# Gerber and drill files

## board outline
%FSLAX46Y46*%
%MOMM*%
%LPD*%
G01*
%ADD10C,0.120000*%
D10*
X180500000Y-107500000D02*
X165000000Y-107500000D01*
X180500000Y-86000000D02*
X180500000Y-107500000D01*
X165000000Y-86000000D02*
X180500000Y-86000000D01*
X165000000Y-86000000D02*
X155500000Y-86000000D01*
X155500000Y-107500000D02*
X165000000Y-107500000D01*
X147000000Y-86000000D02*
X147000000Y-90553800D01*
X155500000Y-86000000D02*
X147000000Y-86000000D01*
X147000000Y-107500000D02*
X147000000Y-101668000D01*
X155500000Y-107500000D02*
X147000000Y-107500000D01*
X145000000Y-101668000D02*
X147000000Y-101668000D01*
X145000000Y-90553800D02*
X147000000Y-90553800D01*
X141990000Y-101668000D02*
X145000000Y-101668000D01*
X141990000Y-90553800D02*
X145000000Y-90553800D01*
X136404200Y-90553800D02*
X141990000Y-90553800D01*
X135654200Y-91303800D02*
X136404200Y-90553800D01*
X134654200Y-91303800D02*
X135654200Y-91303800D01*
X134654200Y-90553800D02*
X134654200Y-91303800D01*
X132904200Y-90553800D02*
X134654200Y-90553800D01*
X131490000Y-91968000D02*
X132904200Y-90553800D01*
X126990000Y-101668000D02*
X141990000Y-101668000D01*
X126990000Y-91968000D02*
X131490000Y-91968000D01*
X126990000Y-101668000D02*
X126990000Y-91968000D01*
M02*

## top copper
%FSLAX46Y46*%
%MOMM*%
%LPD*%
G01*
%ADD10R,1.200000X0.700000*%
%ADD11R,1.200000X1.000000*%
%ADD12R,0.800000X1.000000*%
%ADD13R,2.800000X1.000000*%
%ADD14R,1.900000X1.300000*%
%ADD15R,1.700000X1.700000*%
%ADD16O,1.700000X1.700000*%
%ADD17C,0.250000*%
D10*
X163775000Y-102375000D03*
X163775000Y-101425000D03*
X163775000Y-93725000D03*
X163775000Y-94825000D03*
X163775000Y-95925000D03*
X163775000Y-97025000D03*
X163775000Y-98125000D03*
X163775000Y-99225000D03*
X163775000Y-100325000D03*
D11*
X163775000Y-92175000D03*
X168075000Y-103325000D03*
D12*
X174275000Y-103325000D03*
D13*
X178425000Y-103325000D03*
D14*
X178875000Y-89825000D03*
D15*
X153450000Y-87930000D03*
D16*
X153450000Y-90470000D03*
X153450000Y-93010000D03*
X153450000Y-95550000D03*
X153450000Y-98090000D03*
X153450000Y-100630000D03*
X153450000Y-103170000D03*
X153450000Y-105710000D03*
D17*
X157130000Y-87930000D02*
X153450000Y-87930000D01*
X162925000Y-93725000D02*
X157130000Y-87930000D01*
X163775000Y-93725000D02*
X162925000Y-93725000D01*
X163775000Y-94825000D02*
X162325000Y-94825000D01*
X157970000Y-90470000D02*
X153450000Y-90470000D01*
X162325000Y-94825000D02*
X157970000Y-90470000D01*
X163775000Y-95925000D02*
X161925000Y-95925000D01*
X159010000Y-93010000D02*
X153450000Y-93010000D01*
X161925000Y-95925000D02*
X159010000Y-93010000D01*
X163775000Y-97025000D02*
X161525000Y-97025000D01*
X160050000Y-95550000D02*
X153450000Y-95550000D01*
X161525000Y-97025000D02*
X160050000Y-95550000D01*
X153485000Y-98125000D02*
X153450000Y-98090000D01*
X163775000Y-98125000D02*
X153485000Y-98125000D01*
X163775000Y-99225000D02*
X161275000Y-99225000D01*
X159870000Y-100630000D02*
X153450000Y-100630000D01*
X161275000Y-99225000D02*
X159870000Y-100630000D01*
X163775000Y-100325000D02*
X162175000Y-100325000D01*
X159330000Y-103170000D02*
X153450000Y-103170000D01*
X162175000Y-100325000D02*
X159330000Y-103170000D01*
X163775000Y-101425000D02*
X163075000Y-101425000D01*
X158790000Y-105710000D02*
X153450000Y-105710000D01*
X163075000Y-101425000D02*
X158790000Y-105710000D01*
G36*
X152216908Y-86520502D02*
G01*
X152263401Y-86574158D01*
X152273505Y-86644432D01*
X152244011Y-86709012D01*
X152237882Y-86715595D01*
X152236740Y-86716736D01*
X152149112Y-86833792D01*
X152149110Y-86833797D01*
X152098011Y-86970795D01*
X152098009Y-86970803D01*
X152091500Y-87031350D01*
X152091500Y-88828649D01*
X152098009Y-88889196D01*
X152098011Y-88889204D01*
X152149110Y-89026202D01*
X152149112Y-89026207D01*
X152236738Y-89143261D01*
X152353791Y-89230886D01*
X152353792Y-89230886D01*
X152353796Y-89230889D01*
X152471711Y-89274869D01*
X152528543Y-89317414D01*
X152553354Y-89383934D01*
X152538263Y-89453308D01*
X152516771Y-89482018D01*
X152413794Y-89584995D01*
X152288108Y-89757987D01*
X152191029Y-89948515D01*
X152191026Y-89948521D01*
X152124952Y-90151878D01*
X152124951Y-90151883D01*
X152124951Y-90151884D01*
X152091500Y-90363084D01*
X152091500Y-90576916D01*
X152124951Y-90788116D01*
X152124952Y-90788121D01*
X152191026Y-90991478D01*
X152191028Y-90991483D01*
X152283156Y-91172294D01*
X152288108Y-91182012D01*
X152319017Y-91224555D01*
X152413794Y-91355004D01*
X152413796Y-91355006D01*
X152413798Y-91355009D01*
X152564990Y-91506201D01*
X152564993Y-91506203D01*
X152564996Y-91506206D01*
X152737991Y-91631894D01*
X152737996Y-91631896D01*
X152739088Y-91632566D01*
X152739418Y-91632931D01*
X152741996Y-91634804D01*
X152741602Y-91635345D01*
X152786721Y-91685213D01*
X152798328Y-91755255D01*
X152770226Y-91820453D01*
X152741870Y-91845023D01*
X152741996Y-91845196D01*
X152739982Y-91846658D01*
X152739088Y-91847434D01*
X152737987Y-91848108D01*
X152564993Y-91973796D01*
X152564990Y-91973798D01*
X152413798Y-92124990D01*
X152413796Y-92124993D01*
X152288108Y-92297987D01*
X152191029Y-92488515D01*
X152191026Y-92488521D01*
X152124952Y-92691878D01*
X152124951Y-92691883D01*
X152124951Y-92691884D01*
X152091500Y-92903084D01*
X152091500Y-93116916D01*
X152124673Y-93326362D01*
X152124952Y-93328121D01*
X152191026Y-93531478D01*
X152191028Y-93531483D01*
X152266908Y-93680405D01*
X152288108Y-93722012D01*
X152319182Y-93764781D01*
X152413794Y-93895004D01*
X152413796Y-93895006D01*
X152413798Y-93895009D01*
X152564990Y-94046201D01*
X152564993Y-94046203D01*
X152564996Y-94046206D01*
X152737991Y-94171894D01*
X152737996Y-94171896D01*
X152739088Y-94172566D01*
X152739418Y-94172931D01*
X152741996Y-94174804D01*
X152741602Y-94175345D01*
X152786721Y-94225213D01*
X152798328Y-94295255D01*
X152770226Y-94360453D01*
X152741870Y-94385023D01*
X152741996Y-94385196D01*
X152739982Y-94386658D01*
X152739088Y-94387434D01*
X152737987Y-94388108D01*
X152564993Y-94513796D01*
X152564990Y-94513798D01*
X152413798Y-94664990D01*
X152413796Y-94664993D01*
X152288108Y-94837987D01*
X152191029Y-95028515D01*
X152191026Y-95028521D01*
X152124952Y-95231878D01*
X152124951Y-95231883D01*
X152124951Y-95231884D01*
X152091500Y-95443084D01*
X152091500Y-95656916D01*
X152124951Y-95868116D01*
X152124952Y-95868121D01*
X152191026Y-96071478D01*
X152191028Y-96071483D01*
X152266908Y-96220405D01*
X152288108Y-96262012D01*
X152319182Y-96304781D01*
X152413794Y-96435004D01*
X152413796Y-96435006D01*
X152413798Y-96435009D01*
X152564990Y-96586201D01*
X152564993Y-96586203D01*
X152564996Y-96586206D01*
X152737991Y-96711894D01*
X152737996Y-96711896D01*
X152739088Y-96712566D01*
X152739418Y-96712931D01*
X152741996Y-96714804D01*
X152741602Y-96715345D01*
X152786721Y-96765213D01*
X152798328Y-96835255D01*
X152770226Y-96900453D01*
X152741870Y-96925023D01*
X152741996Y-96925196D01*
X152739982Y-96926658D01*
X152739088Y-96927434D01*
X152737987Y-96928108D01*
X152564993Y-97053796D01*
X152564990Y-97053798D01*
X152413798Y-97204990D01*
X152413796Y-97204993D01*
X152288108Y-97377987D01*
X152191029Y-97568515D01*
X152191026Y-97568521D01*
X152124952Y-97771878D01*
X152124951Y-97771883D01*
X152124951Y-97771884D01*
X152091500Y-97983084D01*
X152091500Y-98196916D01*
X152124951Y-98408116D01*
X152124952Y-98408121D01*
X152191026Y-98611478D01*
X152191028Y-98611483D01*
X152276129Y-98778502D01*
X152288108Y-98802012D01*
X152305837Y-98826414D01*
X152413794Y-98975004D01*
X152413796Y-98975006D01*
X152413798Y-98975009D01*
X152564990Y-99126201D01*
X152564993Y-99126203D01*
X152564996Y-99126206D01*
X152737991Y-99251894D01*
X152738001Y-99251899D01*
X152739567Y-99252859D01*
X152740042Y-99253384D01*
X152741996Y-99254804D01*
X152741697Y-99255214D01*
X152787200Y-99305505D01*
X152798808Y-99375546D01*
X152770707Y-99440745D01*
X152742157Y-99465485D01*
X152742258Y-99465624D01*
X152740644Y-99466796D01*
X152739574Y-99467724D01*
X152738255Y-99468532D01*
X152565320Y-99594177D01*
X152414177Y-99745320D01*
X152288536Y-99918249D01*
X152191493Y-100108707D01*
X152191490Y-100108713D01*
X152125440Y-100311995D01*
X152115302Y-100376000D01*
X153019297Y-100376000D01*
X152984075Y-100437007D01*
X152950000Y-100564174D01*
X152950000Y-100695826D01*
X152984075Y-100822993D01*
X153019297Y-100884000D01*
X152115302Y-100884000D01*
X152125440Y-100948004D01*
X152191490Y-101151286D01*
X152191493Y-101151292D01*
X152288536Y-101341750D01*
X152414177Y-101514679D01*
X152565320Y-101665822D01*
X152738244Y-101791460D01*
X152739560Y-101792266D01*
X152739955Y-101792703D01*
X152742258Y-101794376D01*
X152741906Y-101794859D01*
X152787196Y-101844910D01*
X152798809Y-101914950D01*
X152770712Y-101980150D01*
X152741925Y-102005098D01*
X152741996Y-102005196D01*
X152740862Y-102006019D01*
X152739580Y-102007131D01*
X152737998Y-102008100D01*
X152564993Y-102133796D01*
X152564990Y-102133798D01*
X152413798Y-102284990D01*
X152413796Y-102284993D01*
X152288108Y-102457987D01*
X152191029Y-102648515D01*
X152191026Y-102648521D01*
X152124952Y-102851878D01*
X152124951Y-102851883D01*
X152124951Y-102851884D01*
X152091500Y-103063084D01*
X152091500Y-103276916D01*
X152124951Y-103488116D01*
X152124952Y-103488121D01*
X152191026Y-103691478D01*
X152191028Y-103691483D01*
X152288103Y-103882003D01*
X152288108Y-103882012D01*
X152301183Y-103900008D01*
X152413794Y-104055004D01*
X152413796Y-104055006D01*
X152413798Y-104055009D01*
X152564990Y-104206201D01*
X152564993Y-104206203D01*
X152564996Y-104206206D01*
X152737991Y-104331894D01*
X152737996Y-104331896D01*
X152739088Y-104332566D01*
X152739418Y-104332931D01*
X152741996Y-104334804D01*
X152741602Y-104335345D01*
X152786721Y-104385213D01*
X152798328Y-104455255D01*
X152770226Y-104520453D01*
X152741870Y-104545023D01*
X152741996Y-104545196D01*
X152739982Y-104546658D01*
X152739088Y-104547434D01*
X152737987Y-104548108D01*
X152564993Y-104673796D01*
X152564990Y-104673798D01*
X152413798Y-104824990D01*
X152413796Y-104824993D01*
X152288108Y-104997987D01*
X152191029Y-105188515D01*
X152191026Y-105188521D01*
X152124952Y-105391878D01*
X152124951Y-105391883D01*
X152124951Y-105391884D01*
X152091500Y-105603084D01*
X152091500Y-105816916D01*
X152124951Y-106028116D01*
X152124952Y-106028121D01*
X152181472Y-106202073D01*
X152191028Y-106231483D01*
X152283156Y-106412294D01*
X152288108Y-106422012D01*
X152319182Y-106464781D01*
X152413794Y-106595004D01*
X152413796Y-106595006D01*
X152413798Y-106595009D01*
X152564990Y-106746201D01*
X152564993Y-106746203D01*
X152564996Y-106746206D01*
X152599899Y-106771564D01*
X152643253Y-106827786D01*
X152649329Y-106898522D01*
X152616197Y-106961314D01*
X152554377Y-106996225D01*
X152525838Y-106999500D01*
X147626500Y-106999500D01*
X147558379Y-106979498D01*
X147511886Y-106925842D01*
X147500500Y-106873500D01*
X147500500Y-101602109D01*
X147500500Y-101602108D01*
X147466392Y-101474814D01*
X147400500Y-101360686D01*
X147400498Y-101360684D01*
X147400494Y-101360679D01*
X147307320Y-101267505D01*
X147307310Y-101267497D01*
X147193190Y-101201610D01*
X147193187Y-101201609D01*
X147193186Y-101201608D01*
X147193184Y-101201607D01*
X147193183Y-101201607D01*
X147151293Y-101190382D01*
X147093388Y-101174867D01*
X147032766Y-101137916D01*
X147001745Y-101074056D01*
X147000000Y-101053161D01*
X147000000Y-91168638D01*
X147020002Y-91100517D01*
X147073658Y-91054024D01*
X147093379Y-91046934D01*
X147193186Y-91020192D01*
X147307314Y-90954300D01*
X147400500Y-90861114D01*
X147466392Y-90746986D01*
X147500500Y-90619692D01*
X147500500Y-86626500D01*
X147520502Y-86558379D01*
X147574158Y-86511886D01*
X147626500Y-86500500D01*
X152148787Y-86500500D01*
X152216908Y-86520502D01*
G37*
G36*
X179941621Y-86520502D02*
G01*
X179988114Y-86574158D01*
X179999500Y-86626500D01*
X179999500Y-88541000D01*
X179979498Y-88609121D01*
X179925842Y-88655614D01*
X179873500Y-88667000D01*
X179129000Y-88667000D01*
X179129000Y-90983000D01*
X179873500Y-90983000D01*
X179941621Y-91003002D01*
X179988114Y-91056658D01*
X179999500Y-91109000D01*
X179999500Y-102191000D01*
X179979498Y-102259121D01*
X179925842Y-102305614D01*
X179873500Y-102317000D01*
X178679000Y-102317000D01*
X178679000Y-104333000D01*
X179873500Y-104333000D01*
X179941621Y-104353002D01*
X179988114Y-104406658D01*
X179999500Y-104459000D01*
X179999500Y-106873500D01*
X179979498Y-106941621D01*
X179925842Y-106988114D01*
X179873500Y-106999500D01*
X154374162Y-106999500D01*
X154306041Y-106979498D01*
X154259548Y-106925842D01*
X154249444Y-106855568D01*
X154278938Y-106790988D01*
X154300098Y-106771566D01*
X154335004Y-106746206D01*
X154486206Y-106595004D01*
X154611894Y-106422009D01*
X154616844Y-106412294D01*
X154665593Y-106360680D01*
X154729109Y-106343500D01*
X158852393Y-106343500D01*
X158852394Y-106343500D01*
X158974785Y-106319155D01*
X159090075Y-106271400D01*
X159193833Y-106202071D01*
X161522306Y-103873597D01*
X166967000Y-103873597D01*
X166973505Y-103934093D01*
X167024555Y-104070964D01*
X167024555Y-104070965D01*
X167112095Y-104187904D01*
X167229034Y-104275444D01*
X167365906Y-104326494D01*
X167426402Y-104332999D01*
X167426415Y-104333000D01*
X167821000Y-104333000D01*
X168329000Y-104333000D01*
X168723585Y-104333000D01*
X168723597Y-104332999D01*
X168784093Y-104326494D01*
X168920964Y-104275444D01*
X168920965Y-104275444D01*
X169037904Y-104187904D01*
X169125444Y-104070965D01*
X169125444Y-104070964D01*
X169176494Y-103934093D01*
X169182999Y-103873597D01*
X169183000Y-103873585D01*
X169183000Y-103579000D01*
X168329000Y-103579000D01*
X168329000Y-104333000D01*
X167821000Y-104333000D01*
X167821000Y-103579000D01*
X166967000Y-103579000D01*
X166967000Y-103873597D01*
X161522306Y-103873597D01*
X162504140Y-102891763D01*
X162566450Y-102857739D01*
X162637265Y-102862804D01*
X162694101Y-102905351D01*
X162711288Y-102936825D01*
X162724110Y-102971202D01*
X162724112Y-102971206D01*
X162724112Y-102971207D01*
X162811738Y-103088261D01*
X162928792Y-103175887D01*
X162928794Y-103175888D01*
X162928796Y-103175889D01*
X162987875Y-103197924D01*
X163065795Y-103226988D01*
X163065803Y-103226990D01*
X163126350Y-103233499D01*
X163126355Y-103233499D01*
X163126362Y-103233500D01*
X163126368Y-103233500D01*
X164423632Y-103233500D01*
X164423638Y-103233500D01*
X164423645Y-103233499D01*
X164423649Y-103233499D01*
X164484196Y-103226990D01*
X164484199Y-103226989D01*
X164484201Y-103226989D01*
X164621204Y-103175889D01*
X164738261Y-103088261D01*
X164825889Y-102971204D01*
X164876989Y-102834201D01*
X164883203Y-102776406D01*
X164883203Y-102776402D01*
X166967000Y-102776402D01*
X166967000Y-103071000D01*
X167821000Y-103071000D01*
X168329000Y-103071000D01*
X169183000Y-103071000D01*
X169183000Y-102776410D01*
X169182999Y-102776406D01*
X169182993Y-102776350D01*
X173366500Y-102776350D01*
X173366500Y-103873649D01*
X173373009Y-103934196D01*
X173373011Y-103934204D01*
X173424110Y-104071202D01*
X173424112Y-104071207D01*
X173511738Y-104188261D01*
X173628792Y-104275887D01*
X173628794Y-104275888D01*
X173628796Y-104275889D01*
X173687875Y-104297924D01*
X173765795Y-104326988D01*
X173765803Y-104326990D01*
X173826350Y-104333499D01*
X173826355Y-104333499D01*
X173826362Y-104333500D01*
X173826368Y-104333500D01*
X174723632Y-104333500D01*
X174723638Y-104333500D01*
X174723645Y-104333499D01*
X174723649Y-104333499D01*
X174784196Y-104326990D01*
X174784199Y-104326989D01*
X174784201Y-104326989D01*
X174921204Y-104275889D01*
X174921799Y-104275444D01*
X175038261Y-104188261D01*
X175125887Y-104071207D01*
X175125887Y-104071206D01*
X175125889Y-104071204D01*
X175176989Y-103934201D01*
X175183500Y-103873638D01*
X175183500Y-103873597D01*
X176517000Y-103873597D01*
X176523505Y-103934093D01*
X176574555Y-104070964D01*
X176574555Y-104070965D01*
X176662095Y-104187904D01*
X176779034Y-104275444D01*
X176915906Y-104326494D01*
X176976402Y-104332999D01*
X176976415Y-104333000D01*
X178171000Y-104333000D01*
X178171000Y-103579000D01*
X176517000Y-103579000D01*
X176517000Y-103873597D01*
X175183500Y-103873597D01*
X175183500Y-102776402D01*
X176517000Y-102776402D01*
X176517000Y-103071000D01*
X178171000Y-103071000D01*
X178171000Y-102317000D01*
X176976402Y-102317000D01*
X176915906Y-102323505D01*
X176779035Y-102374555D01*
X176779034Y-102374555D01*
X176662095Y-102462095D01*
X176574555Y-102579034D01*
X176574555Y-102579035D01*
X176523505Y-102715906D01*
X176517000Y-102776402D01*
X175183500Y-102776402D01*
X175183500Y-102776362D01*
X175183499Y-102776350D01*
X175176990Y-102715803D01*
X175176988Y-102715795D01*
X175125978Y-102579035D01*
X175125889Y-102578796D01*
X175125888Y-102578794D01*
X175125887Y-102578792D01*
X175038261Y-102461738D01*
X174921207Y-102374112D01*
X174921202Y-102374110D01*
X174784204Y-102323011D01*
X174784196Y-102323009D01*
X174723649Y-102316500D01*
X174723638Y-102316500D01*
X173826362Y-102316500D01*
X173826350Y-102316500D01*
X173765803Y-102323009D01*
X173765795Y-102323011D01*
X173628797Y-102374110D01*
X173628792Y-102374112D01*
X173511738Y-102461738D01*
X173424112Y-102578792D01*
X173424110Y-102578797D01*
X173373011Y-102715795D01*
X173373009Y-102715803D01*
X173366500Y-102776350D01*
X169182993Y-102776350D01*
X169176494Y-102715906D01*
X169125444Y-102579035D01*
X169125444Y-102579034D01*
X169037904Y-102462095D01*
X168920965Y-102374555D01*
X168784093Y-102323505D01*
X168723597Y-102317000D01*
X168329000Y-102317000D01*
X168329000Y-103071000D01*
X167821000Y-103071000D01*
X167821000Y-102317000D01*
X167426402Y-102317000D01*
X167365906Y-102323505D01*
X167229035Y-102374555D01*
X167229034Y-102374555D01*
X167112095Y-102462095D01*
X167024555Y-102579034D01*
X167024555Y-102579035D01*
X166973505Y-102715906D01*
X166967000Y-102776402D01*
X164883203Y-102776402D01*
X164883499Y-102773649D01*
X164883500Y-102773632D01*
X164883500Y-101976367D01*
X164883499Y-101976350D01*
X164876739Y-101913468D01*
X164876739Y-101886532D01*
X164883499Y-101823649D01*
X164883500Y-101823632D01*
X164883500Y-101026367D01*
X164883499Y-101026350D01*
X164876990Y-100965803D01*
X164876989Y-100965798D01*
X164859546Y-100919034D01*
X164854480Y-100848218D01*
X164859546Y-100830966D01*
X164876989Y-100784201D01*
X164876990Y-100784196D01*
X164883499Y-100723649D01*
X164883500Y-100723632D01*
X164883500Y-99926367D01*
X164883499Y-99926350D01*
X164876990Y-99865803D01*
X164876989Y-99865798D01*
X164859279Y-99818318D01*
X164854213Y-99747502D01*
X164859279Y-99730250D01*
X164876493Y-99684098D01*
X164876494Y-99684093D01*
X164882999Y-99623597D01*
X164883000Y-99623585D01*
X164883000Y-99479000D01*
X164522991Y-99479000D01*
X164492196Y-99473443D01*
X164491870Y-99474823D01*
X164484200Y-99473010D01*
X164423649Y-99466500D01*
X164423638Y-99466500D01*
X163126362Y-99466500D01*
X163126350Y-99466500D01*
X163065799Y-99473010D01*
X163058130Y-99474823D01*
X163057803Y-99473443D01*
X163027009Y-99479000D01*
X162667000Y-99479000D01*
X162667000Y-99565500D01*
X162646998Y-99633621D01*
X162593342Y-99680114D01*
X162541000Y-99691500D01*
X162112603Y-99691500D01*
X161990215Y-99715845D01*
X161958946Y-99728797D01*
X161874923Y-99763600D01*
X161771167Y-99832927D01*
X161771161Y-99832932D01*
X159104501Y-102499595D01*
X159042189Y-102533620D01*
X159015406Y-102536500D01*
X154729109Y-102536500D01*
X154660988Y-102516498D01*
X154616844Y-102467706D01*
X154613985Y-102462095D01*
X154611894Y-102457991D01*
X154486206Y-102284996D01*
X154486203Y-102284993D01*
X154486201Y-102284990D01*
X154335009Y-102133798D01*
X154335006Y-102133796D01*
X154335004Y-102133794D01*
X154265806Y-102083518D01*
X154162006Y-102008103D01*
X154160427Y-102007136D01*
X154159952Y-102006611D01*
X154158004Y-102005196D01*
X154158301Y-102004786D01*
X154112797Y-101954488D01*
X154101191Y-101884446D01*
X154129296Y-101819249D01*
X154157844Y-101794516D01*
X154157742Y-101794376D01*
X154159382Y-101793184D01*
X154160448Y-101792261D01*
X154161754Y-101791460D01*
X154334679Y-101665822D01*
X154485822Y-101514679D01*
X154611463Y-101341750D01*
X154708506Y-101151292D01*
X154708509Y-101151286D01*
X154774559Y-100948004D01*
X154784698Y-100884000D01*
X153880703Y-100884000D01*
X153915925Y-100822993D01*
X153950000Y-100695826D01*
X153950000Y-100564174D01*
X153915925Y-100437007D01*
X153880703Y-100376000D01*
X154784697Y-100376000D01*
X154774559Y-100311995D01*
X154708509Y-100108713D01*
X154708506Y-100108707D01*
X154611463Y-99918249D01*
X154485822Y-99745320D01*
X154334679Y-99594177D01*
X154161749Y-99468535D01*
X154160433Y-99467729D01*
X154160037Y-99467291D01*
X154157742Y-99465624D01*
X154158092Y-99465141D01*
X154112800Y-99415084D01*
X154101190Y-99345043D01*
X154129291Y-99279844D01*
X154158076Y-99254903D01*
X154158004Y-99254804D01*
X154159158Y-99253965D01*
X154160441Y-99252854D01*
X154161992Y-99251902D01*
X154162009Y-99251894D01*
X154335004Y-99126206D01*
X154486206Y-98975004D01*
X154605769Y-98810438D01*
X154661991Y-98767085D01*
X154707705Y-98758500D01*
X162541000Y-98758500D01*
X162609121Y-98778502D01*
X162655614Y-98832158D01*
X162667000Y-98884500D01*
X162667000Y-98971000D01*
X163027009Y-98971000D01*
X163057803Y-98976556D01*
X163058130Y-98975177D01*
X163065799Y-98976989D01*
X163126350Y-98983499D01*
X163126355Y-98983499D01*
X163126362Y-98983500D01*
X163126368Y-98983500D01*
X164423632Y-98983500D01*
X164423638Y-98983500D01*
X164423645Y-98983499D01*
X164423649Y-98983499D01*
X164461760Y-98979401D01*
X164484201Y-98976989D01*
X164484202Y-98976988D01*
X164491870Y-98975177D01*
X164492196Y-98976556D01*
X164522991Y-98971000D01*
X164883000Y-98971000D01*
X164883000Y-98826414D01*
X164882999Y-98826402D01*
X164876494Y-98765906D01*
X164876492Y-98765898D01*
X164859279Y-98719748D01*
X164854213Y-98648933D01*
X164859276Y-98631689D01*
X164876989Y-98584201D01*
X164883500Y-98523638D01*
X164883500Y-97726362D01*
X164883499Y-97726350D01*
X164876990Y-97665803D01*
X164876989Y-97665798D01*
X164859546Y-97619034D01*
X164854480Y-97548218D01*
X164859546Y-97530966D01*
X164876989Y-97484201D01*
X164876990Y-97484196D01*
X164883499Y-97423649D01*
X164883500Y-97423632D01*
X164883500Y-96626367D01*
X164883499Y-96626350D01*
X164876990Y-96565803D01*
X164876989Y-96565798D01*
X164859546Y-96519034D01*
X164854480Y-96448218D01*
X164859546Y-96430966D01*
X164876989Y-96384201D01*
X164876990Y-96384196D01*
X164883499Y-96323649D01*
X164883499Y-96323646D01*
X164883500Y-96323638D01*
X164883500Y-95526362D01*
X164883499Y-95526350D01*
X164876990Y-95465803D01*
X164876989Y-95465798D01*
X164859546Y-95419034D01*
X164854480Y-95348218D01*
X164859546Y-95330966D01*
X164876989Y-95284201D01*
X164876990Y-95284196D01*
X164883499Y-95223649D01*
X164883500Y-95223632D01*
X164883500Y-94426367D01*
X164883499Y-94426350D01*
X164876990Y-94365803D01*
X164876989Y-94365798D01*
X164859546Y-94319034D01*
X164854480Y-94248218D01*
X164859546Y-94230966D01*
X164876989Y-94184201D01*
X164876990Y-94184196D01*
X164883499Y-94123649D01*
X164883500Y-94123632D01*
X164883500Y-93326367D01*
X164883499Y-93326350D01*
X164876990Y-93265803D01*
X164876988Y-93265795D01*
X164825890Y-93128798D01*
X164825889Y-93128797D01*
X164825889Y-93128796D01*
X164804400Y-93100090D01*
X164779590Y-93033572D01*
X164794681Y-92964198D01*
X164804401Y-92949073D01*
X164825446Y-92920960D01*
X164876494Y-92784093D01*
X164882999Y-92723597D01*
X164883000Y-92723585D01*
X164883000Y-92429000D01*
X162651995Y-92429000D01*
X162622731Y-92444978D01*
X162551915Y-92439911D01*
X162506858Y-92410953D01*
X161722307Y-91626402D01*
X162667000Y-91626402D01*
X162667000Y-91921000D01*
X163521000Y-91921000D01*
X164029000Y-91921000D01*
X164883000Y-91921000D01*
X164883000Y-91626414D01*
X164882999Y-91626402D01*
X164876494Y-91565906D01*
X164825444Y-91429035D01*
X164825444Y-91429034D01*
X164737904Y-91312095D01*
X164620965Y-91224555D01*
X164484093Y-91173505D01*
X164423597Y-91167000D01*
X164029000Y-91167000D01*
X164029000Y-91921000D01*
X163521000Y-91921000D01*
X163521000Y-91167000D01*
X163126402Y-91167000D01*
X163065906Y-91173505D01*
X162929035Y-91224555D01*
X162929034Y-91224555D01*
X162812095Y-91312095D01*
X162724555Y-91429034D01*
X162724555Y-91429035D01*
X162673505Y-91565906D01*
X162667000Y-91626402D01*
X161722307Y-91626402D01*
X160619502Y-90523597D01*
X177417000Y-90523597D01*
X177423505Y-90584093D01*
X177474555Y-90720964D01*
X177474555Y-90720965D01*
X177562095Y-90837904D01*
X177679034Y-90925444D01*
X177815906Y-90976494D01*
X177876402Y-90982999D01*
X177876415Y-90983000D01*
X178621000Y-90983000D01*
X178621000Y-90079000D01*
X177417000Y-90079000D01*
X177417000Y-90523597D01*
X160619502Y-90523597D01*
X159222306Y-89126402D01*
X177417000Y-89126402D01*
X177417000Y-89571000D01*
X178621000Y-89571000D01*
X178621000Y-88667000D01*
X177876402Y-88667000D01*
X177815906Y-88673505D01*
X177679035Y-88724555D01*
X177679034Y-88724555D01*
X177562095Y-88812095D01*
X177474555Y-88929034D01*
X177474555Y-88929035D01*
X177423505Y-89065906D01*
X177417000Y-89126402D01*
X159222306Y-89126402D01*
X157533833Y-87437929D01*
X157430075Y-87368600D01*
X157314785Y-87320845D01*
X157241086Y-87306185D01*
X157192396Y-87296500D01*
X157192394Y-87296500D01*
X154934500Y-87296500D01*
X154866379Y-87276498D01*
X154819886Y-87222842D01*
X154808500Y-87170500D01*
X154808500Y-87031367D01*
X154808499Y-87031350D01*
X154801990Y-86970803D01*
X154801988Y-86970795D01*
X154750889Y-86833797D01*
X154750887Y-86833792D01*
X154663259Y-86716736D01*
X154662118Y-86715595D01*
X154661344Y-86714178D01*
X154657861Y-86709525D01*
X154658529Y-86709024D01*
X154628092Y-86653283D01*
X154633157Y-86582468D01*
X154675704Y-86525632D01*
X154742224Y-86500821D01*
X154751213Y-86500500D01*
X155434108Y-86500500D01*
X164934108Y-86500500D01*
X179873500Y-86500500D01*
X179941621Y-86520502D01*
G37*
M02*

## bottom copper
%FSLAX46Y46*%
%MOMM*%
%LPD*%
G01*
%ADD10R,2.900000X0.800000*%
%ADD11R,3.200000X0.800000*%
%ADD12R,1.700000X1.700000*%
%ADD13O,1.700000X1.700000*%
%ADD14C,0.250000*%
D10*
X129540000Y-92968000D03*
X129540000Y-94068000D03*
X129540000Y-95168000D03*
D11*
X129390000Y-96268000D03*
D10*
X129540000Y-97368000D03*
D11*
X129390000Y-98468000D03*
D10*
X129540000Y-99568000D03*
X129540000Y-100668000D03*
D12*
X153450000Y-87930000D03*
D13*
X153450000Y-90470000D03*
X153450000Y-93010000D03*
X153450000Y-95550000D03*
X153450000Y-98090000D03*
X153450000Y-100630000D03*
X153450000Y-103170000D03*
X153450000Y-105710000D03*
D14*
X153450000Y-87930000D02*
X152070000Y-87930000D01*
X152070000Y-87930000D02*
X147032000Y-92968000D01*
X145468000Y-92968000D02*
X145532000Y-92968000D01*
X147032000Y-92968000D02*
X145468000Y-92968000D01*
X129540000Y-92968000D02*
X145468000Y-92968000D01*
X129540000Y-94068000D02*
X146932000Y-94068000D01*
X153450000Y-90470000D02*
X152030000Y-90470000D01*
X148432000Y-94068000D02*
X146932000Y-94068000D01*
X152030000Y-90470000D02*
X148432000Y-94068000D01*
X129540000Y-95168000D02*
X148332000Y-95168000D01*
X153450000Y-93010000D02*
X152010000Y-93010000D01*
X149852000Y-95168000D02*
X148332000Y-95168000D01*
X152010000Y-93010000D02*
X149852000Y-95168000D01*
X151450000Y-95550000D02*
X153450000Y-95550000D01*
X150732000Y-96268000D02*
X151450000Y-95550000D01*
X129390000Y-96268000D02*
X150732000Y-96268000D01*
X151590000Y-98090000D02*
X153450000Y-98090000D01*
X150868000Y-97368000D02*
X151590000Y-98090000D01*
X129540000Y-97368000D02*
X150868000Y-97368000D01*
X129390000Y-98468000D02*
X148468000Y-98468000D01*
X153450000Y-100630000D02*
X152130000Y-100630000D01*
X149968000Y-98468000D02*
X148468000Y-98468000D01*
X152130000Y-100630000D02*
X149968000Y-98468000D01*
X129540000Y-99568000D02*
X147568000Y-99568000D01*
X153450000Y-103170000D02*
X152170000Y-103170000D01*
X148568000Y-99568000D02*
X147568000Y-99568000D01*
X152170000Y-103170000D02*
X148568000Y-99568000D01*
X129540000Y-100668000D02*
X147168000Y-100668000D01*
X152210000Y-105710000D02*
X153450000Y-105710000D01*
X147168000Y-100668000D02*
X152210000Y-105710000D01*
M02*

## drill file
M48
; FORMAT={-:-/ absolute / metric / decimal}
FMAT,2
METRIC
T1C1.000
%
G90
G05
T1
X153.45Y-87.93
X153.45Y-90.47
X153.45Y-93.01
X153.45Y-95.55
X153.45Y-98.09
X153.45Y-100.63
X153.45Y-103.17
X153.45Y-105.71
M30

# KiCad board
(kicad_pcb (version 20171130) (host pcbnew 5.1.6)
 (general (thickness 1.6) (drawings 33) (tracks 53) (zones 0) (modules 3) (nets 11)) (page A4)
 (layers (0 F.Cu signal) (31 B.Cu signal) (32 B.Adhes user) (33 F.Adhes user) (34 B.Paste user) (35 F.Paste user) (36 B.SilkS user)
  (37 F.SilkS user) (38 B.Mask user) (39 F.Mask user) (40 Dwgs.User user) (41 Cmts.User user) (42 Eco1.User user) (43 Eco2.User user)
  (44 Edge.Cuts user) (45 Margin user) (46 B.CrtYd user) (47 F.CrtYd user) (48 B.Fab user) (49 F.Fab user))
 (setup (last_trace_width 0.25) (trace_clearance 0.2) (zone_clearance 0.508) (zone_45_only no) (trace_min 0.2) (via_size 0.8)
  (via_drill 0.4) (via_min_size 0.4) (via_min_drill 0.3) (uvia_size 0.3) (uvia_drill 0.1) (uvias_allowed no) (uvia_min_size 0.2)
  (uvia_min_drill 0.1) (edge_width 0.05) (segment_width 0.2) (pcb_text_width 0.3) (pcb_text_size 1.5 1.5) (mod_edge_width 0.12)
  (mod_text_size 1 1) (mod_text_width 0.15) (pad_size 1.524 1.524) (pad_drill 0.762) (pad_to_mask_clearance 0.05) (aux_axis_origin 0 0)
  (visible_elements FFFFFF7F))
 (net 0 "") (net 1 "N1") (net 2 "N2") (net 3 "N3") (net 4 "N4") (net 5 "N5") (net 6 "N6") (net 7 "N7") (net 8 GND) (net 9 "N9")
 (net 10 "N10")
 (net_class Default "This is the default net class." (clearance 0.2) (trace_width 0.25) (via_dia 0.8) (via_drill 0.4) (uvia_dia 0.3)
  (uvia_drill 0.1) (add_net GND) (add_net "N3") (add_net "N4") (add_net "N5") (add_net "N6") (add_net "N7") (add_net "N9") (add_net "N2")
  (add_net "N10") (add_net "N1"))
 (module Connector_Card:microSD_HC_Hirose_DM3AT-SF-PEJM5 (layer F.Cu) (at 171.5 96.5 90)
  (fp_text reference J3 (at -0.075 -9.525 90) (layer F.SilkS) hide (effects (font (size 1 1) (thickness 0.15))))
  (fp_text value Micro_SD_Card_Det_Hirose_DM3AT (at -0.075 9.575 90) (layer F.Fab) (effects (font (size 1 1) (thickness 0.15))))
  (pad 9 smd rect (at -5.875 -7.725 90) (size 0.7 1.2) (layers F.Cu F.Paste F.Mask) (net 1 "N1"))
  (pad 8 smd rect (at -4.925 -7.725 90) (size 0.7 1.2) (layers F.Cu F.Paste F.Mask) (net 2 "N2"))
  (pad 1 smd rect (at 2.775 -7.725 90) (size 0.7 1.2) (layers F.Cu F.Paste F.Mask) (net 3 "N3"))
  (pad 2 smd rect (at 1.675 -7.725 90) (size 0.7 1.2) (layers F.Cu F.Paste F.Mask) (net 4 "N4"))
  (pad 3 smd rect (at 0.575 -7.725 90) (size 0.7 1.2) (layers F.Cu F.Paste F.Mask) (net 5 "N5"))
  (pad 4 smd rect (at -0.525 -7.725 90) (size 0.7 1.2) (layers F.Cu F.Paste F.Mask) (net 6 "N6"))
  (pad 5 smd rect (at -1.625 -7.725 90) (size 0.7 1.2) (layers F.Cu F.Paste F.Mask) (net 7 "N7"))
  (pad 6 smd rect (at -2.725 -7.725 90) (size 0.7 1.2) (layers F.Cu F.Paste F.Mask) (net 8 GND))
  (pad 7 smd rect (at -3.825 -7.725 90) (size 0.7 1.2) (layers F.Cu F.Paste F.Mask) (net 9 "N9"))
  (pad 11 smd rect (at 4.325 -7.725 90) (size 1 1.2) (layers F.Cu F.Paste F.Mask) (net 8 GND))
  (pad 11 smd rect (at -6.825 -3.425 90) (size 1 1.2) (layers F.Cu F.Paste F.Mask) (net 8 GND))
  (pad 10 smd rect (at -6.825 2.775 90) (size 1 0.8) (layers F.Cu F.Paste F.Mask) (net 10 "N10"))
  (pad 11 smd rect (at -6.825 6.925 90) (size 1 2.8) (layers F.Cu F.Paste F.Mask) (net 8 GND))
  (pad 11 smd rect (at 6.675 7.375 90) (size 1.3 1.9) (layers F.Cu F.Paste F.Mask) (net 8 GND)))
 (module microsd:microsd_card (layer F.Cu) (at 126.99 101.668)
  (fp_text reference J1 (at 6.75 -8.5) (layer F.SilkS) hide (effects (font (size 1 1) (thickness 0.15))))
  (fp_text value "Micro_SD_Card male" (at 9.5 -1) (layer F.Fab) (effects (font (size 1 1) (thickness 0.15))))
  (fp_line (start 9.4142 -11.1142) (end 15 -11.1142) (layer Edge.Cuts) (width 0.12))
  (fp_line (start 8.6642 -10.3642) (end 9.4142 -11.1142) (layer Edge.Cuts) (width 0.12))
  (fp_line (start 7.6642 -10.3642) (end 8.6642 -10.3642) (layer Edge.Cuts) (width 0.12))
  (fp_line (start 7.6642 -11.1142) (end 7.6642 -10.3642) (layer Edge.Cuts) (width 0.12))
  (fp_line (start 5.9142 -11.1142) (end 7.6642 -11.1142) (layer Edge.Cuts) (width 0.12))
  (fp_line (start 4.5 -9.7) (end 5.9142 -11.1142) (layer Edge.Cuts) (width 0.12))
  (fp_line (start 0 0) (end 15 0) (layer Edge.Cuts) (width 0.12))
  (fp_line (start 0 -9.7) (end 4.5 -9.7) (layer Edge.Cuts) (width 0.12))
  (fp_line (start 0 0) (end 0 -9.7) (layer Edge.Cuts) (width 0.12))
  (pad 1 smd rect (at 2.55 -8.7) (size 2.9 0.8) (layers B.Cu B.Paste B.Mask) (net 3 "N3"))
  (pad 2 smd rect (at 2.55 -7.6) (size 2.9 0.8) (layers B.Cu B.Paste B.Mask) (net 4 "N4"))
  (pad 3 smd rect (at 2.55 -6.5) (size 2.9 0.8) (layers B.Cu B.Paste B.Mask) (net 5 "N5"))
  (pad 4 smd rect (at 2.4 -5.4) (size 3.2 0.8) (layers B.Cu B.Paste B.Mask) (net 6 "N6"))
  (pad 5 smd rect (at 2.55 -4.3) (size 2.9 0.8) (layers B.Cu B.Paste B.Mask) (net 7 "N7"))
  (pad 6 smd rect (at 2.4 -3.2) (size 3.2 0.8) (layers B.Cu B.Paste B.Mask) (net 8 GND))
  (pad 7 smd rect (at 2.55 -2.1) (size 2.9 0.8) (layers B.Cu B.Paste B.Mask) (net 9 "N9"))
  (pad 8 smd rect (at 2.55 -1) (size 2.9 0.8) (layers B.Cu B.Paste B.Mask) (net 2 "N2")))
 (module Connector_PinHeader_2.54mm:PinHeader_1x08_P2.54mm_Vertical (layer F.Cu) (at 153.45 87.93)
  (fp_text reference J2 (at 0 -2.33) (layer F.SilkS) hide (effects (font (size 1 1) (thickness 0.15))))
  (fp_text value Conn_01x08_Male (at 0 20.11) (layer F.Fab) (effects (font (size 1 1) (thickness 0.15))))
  (pad 1 thru_hole rect (at 0 0) (size 1.7 1.7) (drill 1) (layers *.Cu *.Mask) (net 3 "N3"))
  (pad 2 thru_hole oval (at 0 2.54) (size 1.7 1.7) (drill 1) (layers *.Cu *.Mask) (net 4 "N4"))
  (pad 3 thru_hole oval (at 0 5.08) (size 1.7 1.7) (drill 1) (layers *.Cu *.Mask) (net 5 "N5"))
  (pad 4 thru_hole oval (at 0 7.62) (size 1.7 1.7) (drill 1) (layers *.Cu *.Mask) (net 6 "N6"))
  (pad 5 thru_hole oval (at 0 10.16) (size 1.7 1.7) (drill 1) (layers *.Cu *.Mask) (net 7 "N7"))
  (pad 6 thru_hole oval (at 0 12.7) (size 1.7 1.7) (drill 1) (layers *.Cu *.Mask) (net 8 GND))
  (pad 7 thru_hole oval (at 0 15.24) (size 1.7 1.7) (drill 1) (layers *.Cu *.Mask) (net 9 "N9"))
  (pad 8 thru_hole oval (at 0 17.78) (size 1.7 1.7) (drill 1) (layers *.Cu *.Mask) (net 2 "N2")))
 (gr_line (start 180.5 107.5) (end 165 107.5) (layer Edge.Cuts) (width 0.12))
 (gr_line (start 180.5 86) (end 180.5 107.5) (layer Edge.Cuts) (width 0.12))
 (gr_line (start 165 86) (end 180.5 86) (layer Edge.Cuts) (width 0.12))
 (gr_line (start 165 86) (end 155.5 86) (layer Edge.Cuts) (width 0.12))
 (gr_line (start 155.5 107.5) (end 165 107.5) (layer Edge.Cuts) (width 0.12))
 (gr_line (start 147 86) (end 147 90.5538) (layer Edge.Cuts) (width 0.12))
 (gr_line (start 155.5 86) (end 147 86) (layer Edge.Cuts) (width 0.12))
 (gr_line (start 147 107.5) (end 147 101.668) (layer Edge.Cuts) (width 0.12))
 (gr_line (start 155.5 107.5) (end 147 107.5) (layer Edge.Cuts) (width 0.12))
 (gr_line (start 145 101.668) (end 147 101.668) (layer Edge.Cuts) (width 0.12))
 (gr_line (start 145 90.5538) (end 147 90.5538) (layer Edge.Cuts) (width 0.12))
 (gr_line (start 141.99 101.668) (end 145 101.668) (layer Edge.Cuts) (width 0.12))
 (gr_line (start 141.99 90.5538) (end 145 90.5538) (layer Edge.Cuts) (width 0.12))
 (segment (start 153.45 87.93) (end 152.07 87.93) (width 0.25) (layer B.Cu) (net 3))
 (segment (start 152.07 87.93) (end 147.032 92.968) (width 0.25) (layer B.Cu) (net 3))
 (segment (start 145.468 92.968) (end 145.532 92.968) (width 0.25) (layer B.Cu) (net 3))
 (segment (start 147.032 92.968) (end 145.468 92.968) (width 0.25) (layer B.Cu) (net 3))
 (segment (start 129.54 92.968) (end 145.468 92.968) (width 0.25) (layer B.Cu) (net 3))
 (segment (start 157.13 87.93) (end 153.45 87.93) (width 0.25) (layer F.Cu) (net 3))
 (segment (start 162.925 93.725) (end 157.13 87.93) (width 0.25) (layer F.Cu) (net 3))
 (segment (start 163.775 93.725) (end 162.925 93.725) (width 0.25) (layer F.Cu) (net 3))
 (segment (start 129.54 94.068) (end 146.932 94.068) (width 0.25) (layer B.Cu) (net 4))
 (segment (start 153.45 90.47) (end 152.03 90.47) (width 0.25) (layer B.Cu) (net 4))
 (segment (start 148.432 94.068) (end 146.932 94.068) (width 0.25) (layer B.Cu) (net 4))
 (segment (start 152.03 90.47) (end 148.432 94.068) (width 0.25) (layer B.Cu) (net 4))
 (segment (start 163.775 94.825) (end 162.325 94.825) (width 0.25) (layer F.Cu) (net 4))
 (segment (start 157.97 90.47) (end 153.45 90.47) (width 0.25) (layer F.Cu) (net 4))
 (segment (start 162.325 94.825) (end 157.97 90.47) (width 0.25) (layer F.Cu) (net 4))
 (segment (start 129.54 95.168) (end 148.332 95.168) (width 0.25) (layer B.Cu) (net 5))
 (segment (start 153.45 93.01) (end 152.01 93.01) (width 0.25) (layer B.Cu) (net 5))
 (segment (start 149.852 95.168) (end 148.332 95.168) (width 0.25) (layer B.Cu) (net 5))
 (segment (start 152.01 93.01) (end 149.852 95.168) (width 0.25) (layer B.Cu) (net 5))
 (segment (start 163.775 95.925) (end 161.925 95.925) (width 0.25) (layer F.Cu) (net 5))
 (segment (start 159.01 93.01) (end 153.45 93.01) (width 0.25) (layer F.Cu) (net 5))
 (segment (start 161.925 95.925) (end 159.01 93.01) (width 0.25) (layer F.Cu) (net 5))
 (segment (start 151.45 95.55) (end 153.45 95.55) (width 0.25) (layer B.Cu) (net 6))
 (segment (start 150.732 96.268) (end 151.45 95.55) (width 0.25) (layer B.Cu) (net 6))
 (segment (start 129.39 96.268) (end 150.732 96.268) (width 0.25) (layer B.Cu) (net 6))
 (segment (start 163.775 97.025) (end 161.525 97.025) (width 0.25) (layer F.Cu) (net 6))
 (segment (start 160.05 95.55) (end 153.45 95.55) (width 0.25) (layer F.Cu) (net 6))
 (segment (start 161.525 97.025) (end 160.05 95.55) (width 0.25) (layer F.Cu) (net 6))
 (segment (start 151.59 98.09) (end 153.45 98.09) (width 0.25) (layer B.Cu) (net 7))
 (segment (start 150.868 97.368) (end 151.59 98.09) (width 0.25) (layer B.Cu) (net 7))
 (segment (start 129.54 97.368) (end 150.868 97.368) (width 0.25) (layer B.Cu) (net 7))
 (segment (start 153.485 98.125) (end 153.45 98.09) (width 0.25) (layer F.Cu) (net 7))
 (segment (start 163.775 98.125) (end 153.485 98.125) (width 0.25) (layer F.Cu) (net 7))
 (segment (start 129.39 98.468) (end 148.468 98.468) (width 0.25) (layer B.Cu) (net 8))
 (segment (start 153.45 100.63) (end 152.13 100.63) (width 0.25) (layer B.Cu) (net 8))
 (segment (start 149.968 98.468) (end 148.468 98.468) (width 0.25) (layer B.Cu) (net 8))
 (segment (start 152.13 100.63) (end 149.968 98.468) (width 0.25) (layer B.Cu) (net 8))
 (segment (start 163.775 99.225) (end 161.275 99.225) (width 0.25) (layer F.Cu) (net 8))
 (segment (start 159.87 100.63) (end 153.45 100.63) (width 0.25) (layer F.Cu) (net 8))
 (segment (start 161.275 99.225) (end 159.87 100.63) (width 0.25) (layer F.Cu) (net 8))
 (segment (start 129.54 99.568) (end 147.568 99.568) (width 0.25) (layer B.Cu) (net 9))
 (segment (start 153.45 103.17) (end 152.17 103.17) (width 0.25) (layer B.Cu) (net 9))
 (segment (start 148.568 99.568) (end 147.568 99.568) (width 0.25) (layer B.Cu) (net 9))
 (segment (start 152.17 103.17) (end 148.568 99.568) (width 0.25) (layer B.Cu) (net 9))
 (segment (start 163.775 100.325) (end 162.175 100.325) (width 0.25) (layer F.Cu) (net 9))
 (segment (start 159.33 103.17) (end 153.45 103.17) (width 0.25) (layer F.Cu) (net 9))
 (segment (start 162.175 100.325) (end 159.33 103.17) (width 0.25) (layer F.Cu) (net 9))
 (segment (start 129.54 100.668) (end 147.168 100.668) (width 0.25) (layer B.Cu) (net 2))
 (segment (start 152.21 105.71) (end 153.45 105.71) (width 0.25) (layer B.Cu) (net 2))
 (segment (start 147.168 100.668) (end 152.21 105.71) (width 0.25) (layer B.Cu) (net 2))
 (segment (start 163.775 101.425) (end 163.075 101.425) (width 0.25) (layer F.Cu) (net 2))
 (segment (start 158.79 105.71) (end 153.45 105.71) (width 0.25) (layer F.Cu) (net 2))
 (segment (start 163.075 101.425) (end 158.79 105.71) (width 0.25) (layer F.Cu) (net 2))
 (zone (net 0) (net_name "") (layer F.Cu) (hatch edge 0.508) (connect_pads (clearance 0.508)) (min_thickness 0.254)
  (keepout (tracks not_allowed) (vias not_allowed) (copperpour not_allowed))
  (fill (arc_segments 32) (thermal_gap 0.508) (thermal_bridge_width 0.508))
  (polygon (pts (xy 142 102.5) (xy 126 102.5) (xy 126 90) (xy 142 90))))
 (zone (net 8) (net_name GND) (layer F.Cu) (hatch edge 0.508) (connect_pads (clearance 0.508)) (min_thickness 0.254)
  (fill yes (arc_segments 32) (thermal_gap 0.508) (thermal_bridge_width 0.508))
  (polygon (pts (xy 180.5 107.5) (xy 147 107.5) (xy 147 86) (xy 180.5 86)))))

